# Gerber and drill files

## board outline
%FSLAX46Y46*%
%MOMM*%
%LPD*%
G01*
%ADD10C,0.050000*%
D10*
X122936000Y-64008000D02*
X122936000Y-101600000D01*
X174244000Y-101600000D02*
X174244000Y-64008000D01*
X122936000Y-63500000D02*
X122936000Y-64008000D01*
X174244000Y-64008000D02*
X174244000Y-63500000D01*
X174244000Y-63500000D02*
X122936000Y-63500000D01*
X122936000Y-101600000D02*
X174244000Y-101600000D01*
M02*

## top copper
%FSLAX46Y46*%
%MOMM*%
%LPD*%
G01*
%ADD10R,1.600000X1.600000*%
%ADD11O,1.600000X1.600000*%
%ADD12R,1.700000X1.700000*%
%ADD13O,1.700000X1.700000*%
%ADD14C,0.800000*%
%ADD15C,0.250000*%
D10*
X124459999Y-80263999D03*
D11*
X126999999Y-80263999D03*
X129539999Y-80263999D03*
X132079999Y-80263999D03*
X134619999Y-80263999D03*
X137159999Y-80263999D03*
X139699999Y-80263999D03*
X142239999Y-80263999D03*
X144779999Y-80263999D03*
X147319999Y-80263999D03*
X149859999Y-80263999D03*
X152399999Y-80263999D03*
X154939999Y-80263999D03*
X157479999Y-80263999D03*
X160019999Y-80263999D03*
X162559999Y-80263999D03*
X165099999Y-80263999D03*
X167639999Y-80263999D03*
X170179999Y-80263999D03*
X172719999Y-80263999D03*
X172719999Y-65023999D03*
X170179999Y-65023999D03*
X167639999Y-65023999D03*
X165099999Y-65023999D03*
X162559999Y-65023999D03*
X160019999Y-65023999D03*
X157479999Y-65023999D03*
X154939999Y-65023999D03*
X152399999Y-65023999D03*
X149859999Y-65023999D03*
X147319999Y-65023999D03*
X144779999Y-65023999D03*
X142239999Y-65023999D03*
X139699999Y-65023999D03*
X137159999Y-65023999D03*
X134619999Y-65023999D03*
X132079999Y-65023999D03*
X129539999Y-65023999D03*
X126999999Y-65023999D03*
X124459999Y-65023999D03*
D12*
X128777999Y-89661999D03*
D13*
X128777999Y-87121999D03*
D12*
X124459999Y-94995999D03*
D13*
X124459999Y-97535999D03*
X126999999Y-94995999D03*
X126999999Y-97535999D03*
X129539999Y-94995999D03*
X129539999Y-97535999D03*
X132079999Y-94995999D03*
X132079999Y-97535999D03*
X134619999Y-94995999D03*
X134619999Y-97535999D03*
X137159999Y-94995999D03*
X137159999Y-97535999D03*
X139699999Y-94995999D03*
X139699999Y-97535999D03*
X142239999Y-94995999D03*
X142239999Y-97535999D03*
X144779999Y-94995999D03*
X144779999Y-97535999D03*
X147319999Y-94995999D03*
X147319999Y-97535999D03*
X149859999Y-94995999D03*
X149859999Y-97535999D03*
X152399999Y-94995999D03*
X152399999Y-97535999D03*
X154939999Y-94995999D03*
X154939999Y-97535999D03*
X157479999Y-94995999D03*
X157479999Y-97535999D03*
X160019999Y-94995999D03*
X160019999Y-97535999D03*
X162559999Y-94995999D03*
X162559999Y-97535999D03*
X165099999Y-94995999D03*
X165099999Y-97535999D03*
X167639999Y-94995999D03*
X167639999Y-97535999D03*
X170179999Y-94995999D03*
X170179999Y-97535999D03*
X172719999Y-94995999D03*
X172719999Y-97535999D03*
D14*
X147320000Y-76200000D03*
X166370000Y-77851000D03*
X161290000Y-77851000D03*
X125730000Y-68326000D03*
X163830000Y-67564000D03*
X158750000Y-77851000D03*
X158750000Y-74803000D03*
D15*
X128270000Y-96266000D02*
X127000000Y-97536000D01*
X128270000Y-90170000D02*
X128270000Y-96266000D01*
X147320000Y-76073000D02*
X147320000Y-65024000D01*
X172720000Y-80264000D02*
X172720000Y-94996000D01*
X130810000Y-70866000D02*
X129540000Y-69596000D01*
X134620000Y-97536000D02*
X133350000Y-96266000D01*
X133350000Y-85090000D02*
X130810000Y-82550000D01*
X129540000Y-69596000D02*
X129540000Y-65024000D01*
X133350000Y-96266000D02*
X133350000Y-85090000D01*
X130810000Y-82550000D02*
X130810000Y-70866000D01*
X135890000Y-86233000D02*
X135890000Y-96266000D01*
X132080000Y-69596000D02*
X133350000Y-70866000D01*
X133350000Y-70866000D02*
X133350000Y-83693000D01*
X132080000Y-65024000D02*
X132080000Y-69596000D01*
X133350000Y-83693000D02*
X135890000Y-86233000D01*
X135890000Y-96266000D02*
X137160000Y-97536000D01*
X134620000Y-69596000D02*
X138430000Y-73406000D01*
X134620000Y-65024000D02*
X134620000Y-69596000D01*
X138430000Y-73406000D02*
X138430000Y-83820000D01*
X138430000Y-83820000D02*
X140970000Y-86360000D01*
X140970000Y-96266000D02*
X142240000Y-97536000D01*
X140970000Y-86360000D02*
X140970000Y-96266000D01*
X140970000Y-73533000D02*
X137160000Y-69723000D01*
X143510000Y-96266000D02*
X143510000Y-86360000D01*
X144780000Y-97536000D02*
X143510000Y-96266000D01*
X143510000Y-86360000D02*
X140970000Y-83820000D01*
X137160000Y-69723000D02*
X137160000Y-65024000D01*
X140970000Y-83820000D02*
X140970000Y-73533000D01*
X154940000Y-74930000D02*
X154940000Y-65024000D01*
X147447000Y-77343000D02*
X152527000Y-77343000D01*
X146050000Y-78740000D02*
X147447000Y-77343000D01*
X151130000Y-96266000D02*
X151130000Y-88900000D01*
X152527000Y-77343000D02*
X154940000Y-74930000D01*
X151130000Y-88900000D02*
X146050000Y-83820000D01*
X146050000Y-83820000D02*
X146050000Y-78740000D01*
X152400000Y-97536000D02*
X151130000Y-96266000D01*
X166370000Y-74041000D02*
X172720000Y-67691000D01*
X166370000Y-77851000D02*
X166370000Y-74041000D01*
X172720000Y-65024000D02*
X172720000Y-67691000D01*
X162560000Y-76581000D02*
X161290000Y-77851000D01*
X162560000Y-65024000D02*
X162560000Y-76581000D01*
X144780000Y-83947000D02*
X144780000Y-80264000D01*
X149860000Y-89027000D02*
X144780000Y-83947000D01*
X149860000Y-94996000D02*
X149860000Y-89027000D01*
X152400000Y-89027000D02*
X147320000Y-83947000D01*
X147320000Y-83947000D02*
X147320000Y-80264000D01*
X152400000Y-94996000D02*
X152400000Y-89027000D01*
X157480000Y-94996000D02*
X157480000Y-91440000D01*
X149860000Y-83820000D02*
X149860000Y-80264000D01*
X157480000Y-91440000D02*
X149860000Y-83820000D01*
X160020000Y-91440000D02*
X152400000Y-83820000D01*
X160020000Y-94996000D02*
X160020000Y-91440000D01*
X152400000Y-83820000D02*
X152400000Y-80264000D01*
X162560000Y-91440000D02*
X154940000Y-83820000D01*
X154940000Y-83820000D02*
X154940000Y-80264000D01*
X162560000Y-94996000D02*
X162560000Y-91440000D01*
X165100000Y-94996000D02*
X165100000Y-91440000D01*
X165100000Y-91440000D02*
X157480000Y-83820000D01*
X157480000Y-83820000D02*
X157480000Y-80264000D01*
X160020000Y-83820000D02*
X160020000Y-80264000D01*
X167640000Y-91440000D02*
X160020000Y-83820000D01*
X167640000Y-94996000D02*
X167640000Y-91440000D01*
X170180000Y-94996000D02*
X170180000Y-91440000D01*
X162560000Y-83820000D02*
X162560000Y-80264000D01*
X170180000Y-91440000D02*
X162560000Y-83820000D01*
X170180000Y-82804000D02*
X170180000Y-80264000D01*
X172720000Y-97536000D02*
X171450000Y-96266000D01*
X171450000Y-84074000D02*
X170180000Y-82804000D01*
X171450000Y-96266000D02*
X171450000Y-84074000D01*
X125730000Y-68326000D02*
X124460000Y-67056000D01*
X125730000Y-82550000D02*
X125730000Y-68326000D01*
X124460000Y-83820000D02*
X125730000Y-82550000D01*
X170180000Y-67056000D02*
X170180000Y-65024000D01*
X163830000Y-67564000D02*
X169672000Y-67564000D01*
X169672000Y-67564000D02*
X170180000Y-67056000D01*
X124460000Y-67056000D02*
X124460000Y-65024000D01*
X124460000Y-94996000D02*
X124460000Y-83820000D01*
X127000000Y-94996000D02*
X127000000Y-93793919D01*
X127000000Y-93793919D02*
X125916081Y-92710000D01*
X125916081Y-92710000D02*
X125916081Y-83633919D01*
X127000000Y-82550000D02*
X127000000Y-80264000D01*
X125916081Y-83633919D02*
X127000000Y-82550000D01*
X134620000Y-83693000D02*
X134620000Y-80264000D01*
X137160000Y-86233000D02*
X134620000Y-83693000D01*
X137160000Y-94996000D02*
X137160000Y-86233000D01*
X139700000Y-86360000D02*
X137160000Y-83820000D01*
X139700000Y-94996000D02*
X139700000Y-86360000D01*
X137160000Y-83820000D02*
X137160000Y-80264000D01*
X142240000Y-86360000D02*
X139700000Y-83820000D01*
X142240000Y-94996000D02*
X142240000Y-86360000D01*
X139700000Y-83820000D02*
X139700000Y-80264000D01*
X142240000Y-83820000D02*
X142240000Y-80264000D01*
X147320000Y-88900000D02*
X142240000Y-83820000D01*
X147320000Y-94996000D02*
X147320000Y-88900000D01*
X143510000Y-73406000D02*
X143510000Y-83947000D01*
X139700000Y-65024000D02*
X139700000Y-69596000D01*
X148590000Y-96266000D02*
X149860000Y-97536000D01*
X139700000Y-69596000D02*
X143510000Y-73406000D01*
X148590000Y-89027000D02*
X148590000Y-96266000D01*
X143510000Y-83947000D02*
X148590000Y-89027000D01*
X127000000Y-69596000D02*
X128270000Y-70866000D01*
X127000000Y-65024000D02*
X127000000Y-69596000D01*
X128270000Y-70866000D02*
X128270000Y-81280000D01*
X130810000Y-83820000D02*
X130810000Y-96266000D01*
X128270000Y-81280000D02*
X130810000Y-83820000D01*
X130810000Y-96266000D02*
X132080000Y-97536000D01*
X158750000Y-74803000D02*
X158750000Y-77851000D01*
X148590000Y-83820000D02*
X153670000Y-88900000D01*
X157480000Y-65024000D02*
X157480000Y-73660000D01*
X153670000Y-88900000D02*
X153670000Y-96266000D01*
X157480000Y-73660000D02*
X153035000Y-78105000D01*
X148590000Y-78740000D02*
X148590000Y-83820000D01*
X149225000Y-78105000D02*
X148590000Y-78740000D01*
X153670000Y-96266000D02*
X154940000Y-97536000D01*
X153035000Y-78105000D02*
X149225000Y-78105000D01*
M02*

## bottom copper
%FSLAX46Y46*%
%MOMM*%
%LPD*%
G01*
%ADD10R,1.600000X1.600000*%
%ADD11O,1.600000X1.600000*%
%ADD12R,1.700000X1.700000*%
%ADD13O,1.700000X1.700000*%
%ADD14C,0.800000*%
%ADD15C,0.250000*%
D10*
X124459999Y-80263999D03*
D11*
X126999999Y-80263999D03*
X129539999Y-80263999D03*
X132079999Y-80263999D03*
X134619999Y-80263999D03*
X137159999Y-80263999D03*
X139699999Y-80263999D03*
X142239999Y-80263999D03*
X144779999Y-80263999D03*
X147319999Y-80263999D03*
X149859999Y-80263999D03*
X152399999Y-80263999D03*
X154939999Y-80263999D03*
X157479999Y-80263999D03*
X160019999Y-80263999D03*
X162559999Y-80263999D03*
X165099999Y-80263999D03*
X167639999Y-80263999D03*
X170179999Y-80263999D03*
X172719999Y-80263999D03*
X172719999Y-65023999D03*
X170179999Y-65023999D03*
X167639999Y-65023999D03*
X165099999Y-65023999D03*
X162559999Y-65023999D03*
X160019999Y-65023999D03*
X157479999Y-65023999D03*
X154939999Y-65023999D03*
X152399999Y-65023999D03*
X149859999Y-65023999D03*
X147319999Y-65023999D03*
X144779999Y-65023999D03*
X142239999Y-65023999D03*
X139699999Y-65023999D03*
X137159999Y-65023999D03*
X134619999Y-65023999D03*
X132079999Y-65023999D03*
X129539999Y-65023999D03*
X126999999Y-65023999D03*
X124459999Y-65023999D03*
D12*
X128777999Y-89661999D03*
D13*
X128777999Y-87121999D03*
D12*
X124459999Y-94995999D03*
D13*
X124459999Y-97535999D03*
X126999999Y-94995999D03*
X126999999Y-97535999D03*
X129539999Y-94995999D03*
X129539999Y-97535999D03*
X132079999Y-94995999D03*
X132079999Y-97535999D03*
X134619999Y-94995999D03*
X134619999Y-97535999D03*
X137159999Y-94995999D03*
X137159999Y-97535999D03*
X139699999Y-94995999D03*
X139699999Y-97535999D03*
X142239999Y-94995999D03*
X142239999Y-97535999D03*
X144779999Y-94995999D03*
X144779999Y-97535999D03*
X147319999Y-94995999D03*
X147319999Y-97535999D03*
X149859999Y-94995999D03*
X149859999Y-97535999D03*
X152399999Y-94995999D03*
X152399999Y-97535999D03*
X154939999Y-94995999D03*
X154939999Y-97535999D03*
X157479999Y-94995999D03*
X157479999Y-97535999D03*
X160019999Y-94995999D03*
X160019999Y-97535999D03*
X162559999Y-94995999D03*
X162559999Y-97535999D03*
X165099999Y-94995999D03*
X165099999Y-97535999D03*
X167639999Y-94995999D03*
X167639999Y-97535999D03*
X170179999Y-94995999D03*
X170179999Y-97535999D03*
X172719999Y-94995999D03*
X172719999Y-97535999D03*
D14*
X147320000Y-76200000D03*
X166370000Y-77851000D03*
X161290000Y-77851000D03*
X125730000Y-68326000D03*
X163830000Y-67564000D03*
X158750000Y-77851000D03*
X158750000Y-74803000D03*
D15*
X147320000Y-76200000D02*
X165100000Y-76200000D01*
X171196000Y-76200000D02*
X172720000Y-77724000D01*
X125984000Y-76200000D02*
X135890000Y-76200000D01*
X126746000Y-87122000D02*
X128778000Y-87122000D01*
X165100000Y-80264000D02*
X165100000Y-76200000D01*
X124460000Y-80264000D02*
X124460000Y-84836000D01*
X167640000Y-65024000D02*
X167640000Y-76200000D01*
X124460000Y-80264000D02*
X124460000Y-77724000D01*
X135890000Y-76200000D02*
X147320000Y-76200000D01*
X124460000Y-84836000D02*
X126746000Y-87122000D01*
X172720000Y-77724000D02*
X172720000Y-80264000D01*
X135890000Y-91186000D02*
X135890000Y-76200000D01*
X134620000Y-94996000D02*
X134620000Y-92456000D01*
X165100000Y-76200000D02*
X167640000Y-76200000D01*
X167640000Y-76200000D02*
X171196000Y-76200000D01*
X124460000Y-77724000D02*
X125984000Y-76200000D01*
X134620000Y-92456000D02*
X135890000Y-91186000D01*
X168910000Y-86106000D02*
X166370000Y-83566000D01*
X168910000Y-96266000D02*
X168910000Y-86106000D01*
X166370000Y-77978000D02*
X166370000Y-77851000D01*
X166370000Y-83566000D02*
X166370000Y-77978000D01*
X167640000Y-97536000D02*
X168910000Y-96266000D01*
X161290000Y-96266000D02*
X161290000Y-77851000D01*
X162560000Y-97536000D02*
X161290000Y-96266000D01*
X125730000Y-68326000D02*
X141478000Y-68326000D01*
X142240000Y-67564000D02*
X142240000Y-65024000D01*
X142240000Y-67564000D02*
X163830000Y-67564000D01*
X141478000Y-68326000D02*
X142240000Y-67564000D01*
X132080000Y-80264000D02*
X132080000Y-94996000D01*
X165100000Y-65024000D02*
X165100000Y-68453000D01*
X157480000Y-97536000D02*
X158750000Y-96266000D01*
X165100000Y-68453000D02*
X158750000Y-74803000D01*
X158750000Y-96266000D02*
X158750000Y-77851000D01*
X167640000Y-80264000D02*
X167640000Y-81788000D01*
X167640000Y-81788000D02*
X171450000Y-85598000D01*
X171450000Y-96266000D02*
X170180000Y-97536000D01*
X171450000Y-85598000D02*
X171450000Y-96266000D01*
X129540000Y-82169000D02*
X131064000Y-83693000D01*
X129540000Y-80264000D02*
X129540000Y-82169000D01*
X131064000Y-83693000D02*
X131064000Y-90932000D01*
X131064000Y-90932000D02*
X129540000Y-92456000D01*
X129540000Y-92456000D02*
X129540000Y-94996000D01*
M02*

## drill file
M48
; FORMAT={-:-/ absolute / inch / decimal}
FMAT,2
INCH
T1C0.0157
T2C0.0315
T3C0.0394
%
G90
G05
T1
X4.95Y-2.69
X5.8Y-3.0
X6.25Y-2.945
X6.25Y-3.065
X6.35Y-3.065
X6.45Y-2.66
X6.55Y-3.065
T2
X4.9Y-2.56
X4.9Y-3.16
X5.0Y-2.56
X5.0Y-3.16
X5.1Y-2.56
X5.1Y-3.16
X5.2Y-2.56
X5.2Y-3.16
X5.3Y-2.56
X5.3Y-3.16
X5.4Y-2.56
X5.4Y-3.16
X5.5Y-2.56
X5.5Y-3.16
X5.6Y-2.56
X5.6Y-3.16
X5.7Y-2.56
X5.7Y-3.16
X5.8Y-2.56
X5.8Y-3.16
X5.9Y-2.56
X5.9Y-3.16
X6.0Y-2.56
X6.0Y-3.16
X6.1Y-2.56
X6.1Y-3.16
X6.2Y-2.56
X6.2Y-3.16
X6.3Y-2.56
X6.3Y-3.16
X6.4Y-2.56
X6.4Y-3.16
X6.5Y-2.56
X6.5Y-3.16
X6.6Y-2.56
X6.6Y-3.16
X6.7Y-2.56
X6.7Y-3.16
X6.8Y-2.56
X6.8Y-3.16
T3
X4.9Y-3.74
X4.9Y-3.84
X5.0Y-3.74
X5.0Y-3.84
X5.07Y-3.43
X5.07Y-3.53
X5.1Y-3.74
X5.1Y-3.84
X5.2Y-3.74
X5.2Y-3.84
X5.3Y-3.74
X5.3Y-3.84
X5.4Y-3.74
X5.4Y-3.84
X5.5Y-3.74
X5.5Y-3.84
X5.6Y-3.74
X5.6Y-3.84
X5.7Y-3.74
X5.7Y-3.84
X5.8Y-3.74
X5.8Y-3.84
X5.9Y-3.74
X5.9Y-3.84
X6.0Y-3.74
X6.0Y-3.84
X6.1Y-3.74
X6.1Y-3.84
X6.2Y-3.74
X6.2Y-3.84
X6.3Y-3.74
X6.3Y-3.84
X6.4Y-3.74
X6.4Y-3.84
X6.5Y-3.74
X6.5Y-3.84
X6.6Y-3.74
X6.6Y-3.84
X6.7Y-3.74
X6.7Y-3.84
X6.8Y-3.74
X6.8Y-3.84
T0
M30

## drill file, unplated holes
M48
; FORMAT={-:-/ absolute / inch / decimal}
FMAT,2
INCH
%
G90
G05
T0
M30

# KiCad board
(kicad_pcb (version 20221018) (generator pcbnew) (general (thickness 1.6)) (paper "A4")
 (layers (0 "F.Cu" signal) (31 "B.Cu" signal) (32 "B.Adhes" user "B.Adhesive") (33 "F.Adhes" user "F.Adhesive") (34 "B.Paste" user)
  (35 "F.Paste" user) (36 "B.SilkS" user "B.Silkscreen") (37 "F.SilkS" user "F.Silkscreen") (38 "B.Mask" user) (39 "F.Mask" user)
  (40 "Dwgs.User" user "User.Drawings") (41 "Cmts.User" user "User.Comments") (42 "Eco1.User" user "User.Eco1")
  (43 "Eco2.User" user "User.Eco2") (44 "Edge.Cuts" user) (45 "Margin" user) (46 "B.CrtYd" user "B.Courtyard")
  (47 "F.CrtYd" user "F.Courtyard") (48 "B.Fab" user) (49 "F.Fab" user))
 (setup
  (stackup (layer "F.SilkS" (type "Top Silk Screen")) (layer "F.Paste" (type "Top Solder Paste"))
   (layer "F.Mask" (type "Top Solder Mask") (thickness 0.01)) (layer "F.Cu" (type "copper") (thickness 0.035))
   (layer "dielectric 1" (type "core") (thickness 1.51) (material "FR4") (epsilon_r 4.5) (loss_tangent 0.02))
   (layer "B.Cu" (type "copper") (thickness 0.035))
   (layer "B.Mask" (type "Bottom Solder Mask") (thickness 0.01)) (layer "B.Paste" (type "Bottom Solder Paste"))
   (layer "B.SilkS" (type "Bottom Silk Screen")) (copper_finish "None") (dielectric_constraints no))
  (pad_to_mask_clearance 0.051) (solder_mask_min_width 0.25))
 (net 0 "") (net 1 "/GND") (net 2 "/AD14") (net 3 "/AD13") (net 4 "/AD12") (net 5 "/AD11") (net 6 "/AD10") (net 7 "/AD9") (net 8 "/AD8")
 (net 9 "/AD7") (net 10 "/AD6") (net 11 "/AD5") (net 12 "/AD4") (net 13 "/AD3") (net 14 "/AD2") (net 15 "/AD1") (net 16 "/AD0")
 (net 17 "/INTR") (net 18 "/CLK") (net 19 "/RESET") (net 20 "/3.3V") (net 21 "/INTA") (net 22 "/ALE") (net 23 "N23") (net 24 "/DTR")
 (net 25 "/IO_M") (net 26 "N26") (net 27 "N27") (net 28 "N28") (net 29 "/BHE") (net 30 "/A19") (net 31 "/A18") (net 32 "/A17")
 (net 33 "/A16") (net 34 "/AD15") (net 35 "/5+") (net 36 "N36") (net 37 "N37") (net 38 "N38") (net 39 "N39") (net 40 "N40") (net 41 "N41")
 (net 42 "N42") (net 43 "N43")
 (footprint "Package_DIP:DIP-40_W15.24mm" (layer "F.Cu") (at 124.46 80.264 90)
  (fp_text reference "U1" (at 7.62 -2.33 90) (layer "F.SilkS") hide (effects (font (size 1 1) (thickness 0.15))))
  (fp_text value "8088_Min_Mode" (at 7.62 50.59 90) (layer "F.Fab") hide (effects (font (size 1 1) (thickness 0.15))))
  (pad "1" thru_hole rect (at 0 0 90) (size 1.6 1.6) (drill 0.8) (layers "*.Cu" "*.Mask") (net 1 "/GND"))
  (pad "2" thru_hole oval (at 0 2.54 90) (size 1.6 1.6) (drill 0.8) (layers "*.Cu" "*.Mask") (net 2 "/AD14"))
  (pad "3" thru_hole oval (at 0 5.08 90) (size 1.6 1.6) (drill 0.8) (layers "*.Cu" "*.Mask") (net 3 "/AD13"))
  (pad "4" thru_hole oval (at 0 7.62 90) (size 1.6 1.6) (drill 0.8) (layers "*.Cu" "*.Mask") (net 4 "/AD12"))
  (pad "5" thru_hole oval (at 0 10.16 90) (size 1.6 1.6) (drill 0.8) (layers "*.Cu" "*.Mask") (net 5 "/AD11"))
  (pad "6" thru_hole oval (at 0 12.7 90) (size 1.6 1.6) (drill 0.8) (layers "*.Cu" "*.Mask") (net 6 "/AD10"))
  (pad "7" thru_hole oval (at 0 15.24 90) (size 1.6 1.6) (drill 0.8) (layers "*.Cu" "*.Mask") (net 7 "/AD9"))
  (pad "8" thru_hole oval (at 0 17.78 90) (size 1.6 1.6) (drill 0.8) (layers "*.Cu" "*.Mask") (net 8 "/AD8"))
  (pad "9" thru_hole oval (at 0 20.32 90) (size 1.6 1.6) (drill 0.8) (layers "*.Cu" "*.Mask") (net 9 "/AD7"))
  (pad "10" thru_hole oval (at 0 22.86 90) (size 1.6 1.6) (drill 0.8) (layers "*.Cu" "*.Mask") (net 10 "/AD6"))
  (pad "11" thru_hole oval (at 0 25.4 90) (size 1.6 1.6) (drill 0.8) (layers "*.Cu" "*.Mask") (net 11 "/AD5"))
  (pad "12" thru_hole oval (at 0 27.94 90) (size 1.6 1.6) (drill 0.8) (layers "*.Cu" "*.Mask") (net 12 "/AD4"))
  (pad "13" thru_hole oval (at 0 30.48 90) (size 1.6 1.6) (drill 0.8) (layers "*.Cu" "*.Mask") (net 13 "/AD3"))
  (pad "14" thru_hole oval (at 0 33.02 90) (size 1.6 1.6) (drill 0.8) (layers "*.Cu" "*.Mask") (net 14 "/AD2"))
  (pad "15" thru_hole oval (at 0 35.56 90) (size 1.6 1.6) (drill 0.8) (layers "*.Cu" "*.Mask") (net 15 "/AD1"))
  (pad "16" thru_hole oval (at 0 38.1 90) (size 1.6 1.6) (drill 0.8) (layers "*.Cu" "*.Mask") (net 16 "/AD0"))
  (pad "17" thru_hole oval (at 0 40.64 90) (size 1.6 1.6) (drill 0.8) (layers "*.Cu" "*.Mask") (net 1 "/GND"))
  (pad "18" thru_hole oval (at 0 43.18 90) (size 1.6 1.6) (drill 0.8) (layers "*.Cu" "*.Mask") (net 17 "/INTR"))
  (pad "19" thru_hole oval (at 0 45.72 90) (size 1.6 1.6) (drill 0.8) (layers "*.Cu" "*.Mask") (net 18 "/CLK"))
  (pad "20" thru_hole oval (at 0 48.26 90) (size 1.6 1.6) (drill 0.8) (layers "*.Cu" "*.Mask") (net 1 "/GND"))
  (pad "21" thru_hole oval (at 15.24 48.26 90) (size 1.6 1.6) (drill 0.8) (layers "*.Cu" "*.Mask") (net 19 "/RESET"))
  (pad "22" thru_hole oval (at 15.24 45.72 90) (size 1.6 1.6) (drill 0.8) (layers "*.Cu" "*.Mask") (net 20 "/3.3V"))
  (pad "23" thru_hole oval (at 15.24 43.18 90) (size 1.6 1.6) (drill 0.8) (layers "*.Cu" "*.Mask") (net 1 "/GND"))
  (pad "24" thru_hole oval (at 15.24 40.64 90) (size 1.6 1.6) (drill 0.8) (layers "*.Cu" "*.Mask") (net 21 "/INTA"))
  (pad "25" thru_hole oval (at 15.24 38.1 90) (size 1.6 1.6) (drill 0.8) (layers "*.Cu" "*.Mask") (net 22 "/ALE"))
  (pad "26" thru_hole oval (at 15.24 35.56 90) (size 1.6 1.6) (drill 0.8) (layers "*.Cu" "*.Mask") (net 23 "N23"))
  (pad "27" thru_hole oval (at 15.24 33.02 90) (size 1.6 1.6) (drill 0.8) (layers "*.Cu" "*.Mask") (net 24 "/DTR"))
  (pad "28" thru_hole oval (at 15.24 30.48 90) (size 1.6 1.6) (drill 0.8) (layers "*.Cu" "*.Mask") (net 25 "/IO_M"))
  (pad "29" thru_hole oval (at 15.24 27.94 90) (size 1.6 1.6) (drill 0.8) (layers "*.Cu" "*.Mask") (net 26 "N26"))
  (pad "30" thru_hole oval (at 15.24 25.4 90) (size 1.6 1.6) (drill 0.8) (layers "*.Cu" "*.Mask") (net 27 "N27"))
  (pad "31" thru_hole oval (at 15.24 22.86 90) (size 1.6 1.6) (drill 0.8) (layers "*.Cu" "*.Mask") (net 1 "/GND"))
  (pad "32" thru_hole oval (at 15.24 20.32 90) (size 1.6 1.6) (drill 0.8) (layers "*.Cu" "*.Mask") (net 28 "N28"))
  (pad "33" thru_hole oval (at 15.24 17.78 90) (size 1.6 1.6) (drill 0.8) (layers "*.Cu" "*.Mask") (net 20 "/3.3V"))
  (pad "34" thru_hole oval (at 15.24 15.24 90) (size 1.6 1.6) (drill 0.8) (layers "*.Cu" "*.Mask") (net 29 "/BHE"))
  (pad "35" thru_hole oval (at 15.24 12.7 90) (size 1.6 1.6) (drill 0.8) (layers "*.Cu" "*.Mask") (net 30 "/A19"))
  (pad "36" thru_hole oval (at 15.24 10.16 90) (size 1.6 1.6) (drill 0.8) (layers "*.Cu" "*.Mask") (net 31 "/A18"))
  (pad "37" thru_hole oval (at 15.24 7.62 90) (size 1.6 1.6) (drill 0.8) (layers "*.Cu" "*.Mask") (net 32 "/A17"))
  (pad "38" thru_hole oval (at 15.24 5.08 90) (size 1.6 1.6) (drill 0.8) (layers "*.Cu" "*.Mask") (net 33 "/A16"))
  (pad "39" thru_hole oval (at 15.24 2.54 90) (size 1.6 1.6) (drill 0.8) (layers "*.Cu" "*.Mask") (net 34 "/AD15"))
  (pad "40" thru_hole oval (at 15.24 0 90) (size 1.6 1.6) (drill 0.8) (layers "*.Cu" "*.Mask") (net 20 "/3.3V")))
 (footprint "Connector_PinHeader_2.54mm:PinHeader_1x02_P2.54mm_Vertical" (layer "F.Cu") (at 128.778 89.662 180)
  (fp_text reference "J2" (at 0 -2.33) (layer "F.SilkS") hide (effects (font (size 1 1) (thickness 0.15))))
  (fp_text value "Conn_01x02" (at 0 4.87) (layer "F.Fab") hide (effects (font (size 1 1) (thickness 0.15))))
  (pad "1" thru_hole rect (at 0 0 180) (size 1.7 1.7) (drill 1) (layers "*.Cu" "*.Mask") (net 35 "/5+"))
  (pad "2" thru_hole oval (at 0 2.54 180) (size 1.7 1.7) (drill 1) (layers "*.Cu" "*.Mask") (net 1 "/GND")))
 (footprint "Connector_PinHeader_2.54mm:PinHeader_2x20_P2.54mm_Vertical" (layer "B.Cu") (at 124.46 94.996 -90)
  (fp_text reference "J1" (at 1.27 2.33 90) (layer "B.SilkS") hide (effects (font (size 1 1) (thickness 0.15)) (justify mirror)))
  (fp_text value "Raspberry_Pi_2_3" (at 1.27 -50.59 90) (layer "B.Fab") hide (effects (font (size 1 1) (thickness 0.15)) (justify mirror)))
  (pad "1" thru_hole rect (at 0 0 270) (size 1.7 1.7) (drill 1) (layers "*.Cu" "*.Mask") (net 20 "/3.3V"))
  (pad "2" thru_hole oval (at 2.54 0 270) (size 1.7 1.7) (drill 1) (layers "*.Cu" "*.Mask") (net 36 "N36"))
  (pad "3" thru_hole oval (at 0 -2.54 270) (size 1.7 1.7) (drill 1) (layers "*.Cu" "*.Mask") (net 2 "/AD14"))
  (pad "4" thru_hole oval (at 2.54 -2.54 270) (size 1.7 1.7) (drill 1) (layers "*.Cu" "*.Mask") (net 35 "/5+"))
  (pad "5" thru_hole oval (at 0 -5.08 270) (size 1.7 1.7) (drill 1) (layers "*.Cu" "*.Mask") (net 3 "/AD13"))
  (pad "6" thru_hole oval (at 2.54 -5.08 270) (size 1.7 1.7) (drill 1) (layers "*.Cu" "*.Mask") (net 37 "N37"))
  (pad "7" thru_hole oval (at 0 -7.62 270) (size 1.7 1.7) (drill 1) (layers "*.Cu" "*.Mask") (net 4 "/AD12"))
  (pad "8" thru_hole oval (at 2.54 -7.62 270) (size 1.7 1.7) (drill 1) (layers "*.Cu" "*.Mask") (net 34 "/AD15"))
  (pad "9" thru_hole oval (at 0 -10.16 270) (size 1.7 1.7) (drill 1) (layers "*.Cu" "*.Mask") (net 1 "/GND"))
  (pad "10" thru_hole oval (at 2.54 -10.16 270) (size 1.7 1.7) (drill 1) (layers "*.Cu" "*.Mask") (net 33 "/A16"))
  (pad "11" thru_hole oval (at 0 -12.7 270) (size 1.7 1.7) (drill 1) (layers "*.Cu" "*.Mask") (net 5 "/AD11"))
  (pad "12" thru_hole oval (at 2.54 -12.7 270) (size 1.7 1.7) (drill 1) (layers "*.Cu" "*.Mask") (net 32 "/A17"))
  (pad "13" thru_hole oval (at 0 -15.24 270) (size 1.7 1.7) (drill 1) (layers "*.Cu" "*.Mask") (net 6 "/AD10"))
  (pad "14" thru_hole oval (at 2.54 -15.24 270) (size 1.7 1.7) (drill 1) (layers "*.Cu" "*.Mask") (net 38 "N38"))
  (pad "15" thru_hole oval (at 0 -17.78 270) (size 1.7 1.7) (drill 1) (layers "*.Cu" "*.Mask") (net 7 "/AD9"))
  (pad "16" thru_hole oval (at 2.54 -17.78 270) (size 1.7 1.7) (drill 1) (layers "*.Cu" "*.Mask") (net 31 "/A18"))
  (pad "17" thru_hole oval (at 0 -20.32 270) (size 1.7 1.7) (drill 1) (layers "*.Cu" "*.Mask") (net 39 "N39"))
  (pad "18" thru_hole oval (at 2.54 -20.32 270) (size 1.7 1.7) (drill 1) (layers "*.Cu" "*.Mask") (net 30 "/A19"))
  (pad "19" thru_hole oval (at 0 -22.86 270) (size 1.7 1.7) (drill 1) (layers "*.Cu" "*.Mask") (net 8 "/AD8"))
  (pad "20" thru_hole oval (at 2.54 -22.86 270) (size 1.7 1.7) (drill 1) (layers "*.Cu" "*.Mask") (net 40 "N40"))
  (pad "21" thru_hole oval (at 0 -25.4 270) (size 1.7 1.7) (drill 1) (layers "*.Cu" "*.Mask") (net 9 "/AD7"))
  (pad "22" thru_hole oval (at 2.54 -25.4 270) (size 1.7 1.7) (drill 1) (layers "*.Cu" "*.Mask") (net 29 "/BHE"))
  (pad "23" thru_hole oval (at 0 -27.94 270) (size 1.7 1.7) (drill 1) (layers "*.Cu" "*.Mask") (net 10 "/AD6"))
  (pad "24" thru_hole oval (at 2.54 -27.94 270) (size 1.7 1.7) (drill 1) (layers "*.Cu" "*.Mask") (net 25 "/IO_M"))
  (pad "25" thru_hole oval (at 0 -30.48 270) (size 1.7 1.7) (drill 1) (layers "*.Cu" "*.Mask") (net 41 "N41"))
  (pad "26" thru_hole oval (at 2.54 -30.48 270) (size 1.7 1.7) (drill 1) (layers "*.Cu" "*.Mask") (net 24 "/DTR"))
  (pad "27" thru_hole oval (at 0 -33.02 270) (size 1.7 1.7) (drill 1) (layers "*.Cu" "*.Mask") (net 11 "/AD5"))
  (pad "28" thru_hole oval (at 2.54 -33.02 270) (size 1.7 1.7) (drill 1) (layers "*.Cu" "*.Mask") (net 21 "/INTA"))
  (pad "29" thru_hole oval (at 0 -35.56 270) (size 1.7 1.7) (drill 1) (layers "*.Cu" "*.Mask") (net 12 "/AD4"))
  (pad "30" thru_hole oval (at 2.54 -35.56 270) (size 1.7 1.7) (drill 1) (layers "*.Cu" "*.Mask") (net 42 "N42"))
  (pad "31" thru_hole oval (at 0 -38.1 270) (size 1.7 1.7) (drill 1) (layers "*.Cu" "*.Mask") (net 13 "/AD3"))
  (pad "32" thru_hole oval (at 2.54 -38.1 270) (size 1.7 1.7) (drill 1) (layers "*.Cu" "*.Mask") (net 22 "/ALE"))
  (pad "33" thru_hole oval (at 0 -40.64 270) (size 1.7 1.7) (drill 1) (layers "*.Cu" "*.Mask") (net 14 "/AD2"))
  (pad "34" thru_hole oval (at 2.54 -40.64 270) (size 1.7 1.7) (drill 1) (layers "*.Cu" "*.Mask") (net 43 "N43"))
  (pad "35" thru_hole oval (at 0 -43.18 270) (size 1.7 1.7) (drill 1) (layers "*.Cu" "*.Mask") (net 15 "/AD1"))
  (pad "36" thru_hole oval (at 2.54 -43.18 270) (size 1.7 1.7) (drill 1) (layers "*.Cu" "*.Mask") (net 19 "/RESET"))
  (pad "37" thru_hole oval (at 0 -45.72 270) (size 1.7 1.7) (drill 1) (layers "*.Cu" "*.Mask") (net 16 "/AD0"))
  (pad "38" thru_hole oval (at 2.54 -45.72 270) (size 1.7 1.7) (drill 1) (layers "*.Cu" "*.Mask") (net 17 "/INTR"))
  (pad "39" thru_hole oval (at 0 -48.26 270) (size 1.7 1.7) (drill 1) (layers "*.Cu" "*.Mask") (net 1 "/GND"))
  (pad "40" thru_hole oval (at 2.54 -48.26 270) (size 1.7 1.7) (drill 1) (layers "*.Cu" "*.Mask") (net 18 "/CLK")))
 (gr_line (start 122.936 64.008) (end 122.936 101.6) (stroke (width 0.05) (type solid)) (layer "Edge.Cuts"))
 (gr_line (start 174.244 101.6) (end 174.244 64.008) (stroke (width 0.05) (type solid)) (layer "Edge.Cuts"))
 (gr_line (start 122.936 63.5) (end 122.936 64.008) (stroke (width 0.05) (type solid)) (layer "Edge.Cuts"))
 (gr_line (start 174.244 64.008) (end 174.244 63.5) (stroke (width 0.05) (type solid)) (layer "Edge.Cuts"))
 (gr_line (start 174.244 63.5) (end 122.936 63.5) (stroke (width 0.05) (type solid)) (layer "Edge.Cuts"))
 (gr_line (start 122.936 101.6) (end 174.244 101.6) (stroke (width 0.05) (type solid)) (layer "Edge.Cuts"))
 (segment (start 128.27 96.266) (end 127 97.536) (width 0.25) (layer "F.Cu") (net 35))
 (segment (start 128.27 90.17) (end 128.27 96.266) (width 0.25) (layer "F.Cu") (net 35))
 (segment (start 147.32 76.073) (end 147.32 65.024) (width 0.25) (layer "F.Cu") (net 1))
 (segment (start 172.72 80.264) (end 172.72 94.996) (width 0.25) (layer "F.Cu") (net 1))
 (via (at 147.32 76.2) (size 0.8) (drill 0.4) (layers "F.Cu" "B.Cu") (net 1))
 (segment (start 147.32 76.2) (end 165.1 76.2) (width 0.25) (layer "B.Cu") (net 1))
 (segment (start 171.196 76.2) (end 172.72 77.724) (width 0.25) (layer "B.Cu") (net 1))
 (segment (start 125.984 76.2) (end 135.89 76.2) (width 0.25) (layer "B.Cu") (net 1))
 (segment (start 126.746 87.122) (end 128.778 87.122) (width 0.25) (layer "B.Cu") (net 1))
 (segment (start 165.1 80.264) (end 165.1 76.2) (width 0.25) (layer "B.Cu") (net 1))
 (segment (start 124.46 80.264) (end 124.46 84.836) (width 0.25) (layer "B.Cu") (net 1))
 (segment (start 167.64 65.024) (end 167.64 76.2) (width 0.25) (layer "B.Cu") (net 1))
 (segment (start 124.46 80.264) (end 124.46 77.724) (width 0.25) (layer "B.Cu") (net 1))
 (segment (start 135.89 76.2) (end 147.32 76.2) (width 0.25) (layer "B.Cu") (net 1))
 (segment (start 124.46 84.836) (end 126.746 87.122) (width 0.25) (layer "B.Cu") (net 1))
 (segment (start 172.72 77.724) (end 172.72 80.264) (width 0.25) (layer "B.Cu") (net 1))
 (segment (start 135.89 91.186) (end 135.89 76.2) (width 0.25) (layer "B.Cu") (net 1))
 (segment (start 134.62 94.996) (end 134.62 92.456) (width 0.25) (layer "B.Cu") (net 1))
 (segment (start 165.1 76.2) (end 167.64 76.2) (width 0.25) (layer "B.Cu") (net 1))
 (segment (start 167.64 76.2) (end 171.196 76.2) (width 0.25) (layer "B.Cu") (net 1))
 (segment (start 124.46 77.724) (end 125.984 76.2) (width 0.25) (layer "B.Cu") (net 1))
 (segment (start 134.62 92.456) (end 135.89 91.186) (width 0.25) (layer "B.Cu") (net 1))
 (segment (start 130.81 70.866) (end 129.54 69.596) (width 0.25) (layer "F.Cu") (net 33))
 (segment (start 134.62 97.536) (end 133.35 96.266) (width 0.25) (layer "F.Cu") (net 33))
 (segment (start 133.35 85.09) (end 130.81 82.55) (width 0.25) (layer "F.Cu") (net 33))
 (segment (start 129.54 69.596) (end 129.54 65.024) (width 0.25) (layer "F.Cu") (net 33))
 (segment (start 133.35 96.266) (end 133.35 85.09) (width 0.25) (layer "F.Cu") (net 33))
 (segment (start 130.81 82.55) (end 130.81 70.866) (width 0.25) (layer "F.Cu") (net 33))
 (segment (start 135.89 86.233) (end 135.89 96.266) (width 0.25) (layer "F.Cu") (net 32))
 (segment (start 132.08 69.596) (end 133.35 70.866) (width 0.25) (layer "F.Cu") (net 32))
 (segment (start 133.35 70.866) (end 133.35 83.693) (width 0.25) (layer "F.Cu") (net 32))
 (segment (start 132.08 65.024) (end 132.08 69.596) (width 0.25) (layer "F.Cu") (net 32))
 (segment (start 133.35 83.693) (end 135.89 86.233) (width 0.25) (layer "F.Cu") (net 32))
 (segment (start 135.89 96.266) (end 137.16 97.536) (width 0.25) (layer "F.Cu") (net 32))
 (segment (start 134.62 69.596) (end 138.43 73.406) (width 0.25) (layer "F.Cu") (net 31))
 (segment (start 134.62 65.024) (end 134.62 69.596) (width 0.25) (layer "F.Cu") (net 31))
 (segment (start 138.43 73.406) (end 138.43 83.82) (width 0.25) (layer "F.Cu") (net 31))
 (segment (start 138.43 83.82) (end 140.97 86.36) (width 0.25) (layer "F.Cu") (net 31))
 (segment (start 140.97 96.266) (end 142.24 97.536) (width 0.25) (layer "F.Cu") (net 31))
 (segment (start 140.97 86.36) (end 140.97 96.266) (width 0.25) (layer "F.Cu") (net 31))
 (segment (start 140.97 73.533) (end 137.16 69.723) (width 0.25) (layer "F.Cu") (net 30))
 (segment (start 143.51 96.266) (end 143.51 86.36) (width 0.25) (layer "F.Cu") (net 30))
 (segment (start 144.78 97.536) (end 143.51 96.266) (width 0.25) (layer "F.Cu") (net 30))
 (segment (start 143.51 86.36) (end 140.97 83.82) (width 0.25) (layer "F.Cu") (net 30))
 (segment (start 137.16 69.723) (end 137.16 65.024) (width 0.25) (layer "F.Cu") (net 30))
 (segment (start 140.97 83.82) (end 140.97 73.533) (width 0.25) (layer "F.Cu") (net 30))
 (segment (start 154.94 74.93) (end 154.94 65.024) (width 0.25) (layer "F.Cu") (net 25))
 (segment (start 147.447 77.343) (end 152.527 77.343) (width 0.25) (layer "F.Cu") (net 25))
 (segment (start 146.05 78.74) (end 147.447 77.343) (width 0.25) (layer "F.Cu") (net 25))
 (segment (start 151.13 96.266) (end 151.13 88.9) (width 0.25) (layer "F.Cu") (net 25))
 (segment (start 152.527 77.343) (end 154.94 74.93) (width 0.25) (layer "F.Cu") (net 25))
 (segment (start 151.13 88.9) (end 146.05 83.82) (width 0.25) (layer "F.Cu") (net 25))
 (segment (start 146.05 83.82) (end 146.05 78.74) (width 0.25) (layer "F.Cu") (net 25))
 (segment (start 152.4 97.536) (end 151.13 96.266) (width 0.25) (layer "F.Cu") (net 25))
 (segment (start 166.37 74.041) (end 172.72 67.691) (width 0.25) (layer "F.Cu") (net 19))
 (segment (start 166.37 77.851) (end 166.37 74.041) (width 0.25) (layer "F.Cu") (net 19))
 (segment (start 172.72 65.024) (end 172.72 67.691) (width 0.25) (layer "F.Cu") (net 19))
 (via (at 166.37 77.851) (size 0.8) (drill 0.4) (layers "F.Cu" "B.Cu") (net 19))
 (segment (start 168.91 86.106) (end 166.37 83.566) (width 0.25) (layer "B.Cu") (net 19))
 (segment (start 168.91 96.266) (end 168.91 86.106) (width 0.25) (layer "B.Cu") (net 19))
 (segment (start 166.37 77.978) (end 166.37 77.851) (width 0.25) (layer "B.Cu") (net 19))
 (segment (start 166.37 83.566) (end 166.37 77.978) (width 0.25) (layer "B.Cu") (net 19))
 (segment (start 167.64 97.536) (end 168.91 96.266) (width 0.25) (layer "B.Cu") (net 19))
 (segment (start 162.56 76.581) (end 161.29 77.851) (width 0.25) (layer "F.Cu") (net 22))
 (segment (start 162.56 65.024) (end 162.56 76.581) (width 0.25) (layer "F.Cu") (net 22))
 (via (at 161.29 77.851) (size 0.8) (drill 0.4) (layers "F.Cu" "B.Cu") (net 22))
 (segment (start 161.29 96.266) (end 161.29 77.851) (width 0.25) (layer "B.Cu") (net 22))
 (segment (start 162.56 97.536) (end 161.29 96.266) (width 0.25) (layer "B.Cu") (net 22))
 (segment (start 144.78 83.947) (end 144.78 80.264) (width 0.25) (layer "F.Cu") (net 9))
 (segment (start 149.86 89.027) (end 144.78 83.947) (width 0.25) (layer "F.Cu") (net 9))
 (segment (start 149.86 94.996) (end 149.86 89.027) (width 0.25) (layer "F.Cu") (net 9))
 (segment (start 152.4 89.027) (end 147.32 83.947) (width 0.25) (layer "F.Cu") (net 10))
 (segment (start 147.32 83.947) (end 147.32 80.264) (width 0.25) (layer "F.Cu") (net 10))
 (segment (start 152.4 94.996) (end 152.4 89.027) (width 0.25) (layer "F.Cu") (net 10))
 (segment (start 157.48 94.996) (end 157.48 91.44) (width 0.25) (layer "F.Cu") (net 11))
 (segment (start 149.86 83.82) (end 149.86 80.264) (width 0.25) (layer "F.Cu") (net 11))
 (segment (start 157.48 91.44) (end 149.86 83.82) (width 0.25) (layer "F.Cu") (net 11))
 (segment (start 160.02 91.44) (end 152.4 83.82) (width 0.25) (layer "F.Cu") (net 12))
 (segment (start 160.02 94.996) (end 160.02 91.44) (width 0.25) (layer "F.Cu") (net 12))
 (segment (start 152.4 83.82) (end 152.4 80.264) (width 0.25) (layer "F.Cu") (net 12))
 (segment (start 162.56 91.44) (end 154.94 83.82) (width 0.25) (layer "F.Cu") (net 13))
 (segment (start 154.94 83.82) (end 154.94 80.264) (width 0.25) (layer "F.Cu") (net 13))
 (segment (start 162.56 94.996) (end 162.56 91.44) (width 0.25) (layer "F.Cu") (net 13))
 (segment (start 165.1 94.996) (end 165.1 91.44) (width 0.25) (layer "F.Cu") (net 14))
 (segment (start 165.1 91.44) (end 157.48 83.82) (width 0.25) (layer "F.Cu") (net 14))
 (segment (start 157.48 83.82) (end 157.48 80.264) (width 0.25) (layer "F.Cu") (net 14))
 (segment (start 160.02 83.82) (end 160.02 80.264) (width 0.25) (layer "F.Cu") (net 15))
 (segment (start 167.64 91.44) (end 160.02 83.82) (width 0.25) (layer "F.Cu") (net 15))
 (segment (start 167.64 94.996) (end 167.64 91.44) (width 0.25) (layer "F.Cu") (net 15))
 (segment (start 170.18 94.996) (end 170.18 91.44) (width 0.25) (layer "F.Cu") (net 16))
 (segment (start 162.56 83.82) (end 162.56 80.264) (width 0.25) (layer "F.Cu") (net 16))
 (segment (start 170.18 91.44) (end 162.56 83.82) (width 0.25) (layer "F.Cu") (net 16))
 (segment (start 170.18 82.804) (end 170.18 80.264) (width 0.25) (layer "F.Cu") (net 18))
 (segment (start 172.72 97.536) (end 171.45 96.266) (width 0.25) (layer "F.Cu") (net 18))
 (segment (start 171.45 84.074) (end 170.18 82.804) (width 0.25) (layer "F.Cu") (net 18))
 (segment (start 171.45 96.266) (end 171.45 84.074) (width 0.25) (layer "F.Cu") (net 18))
 (segment (start 125.73 68.326) (end 124.46 67.056) (width 0.25) (layer "F.Cu") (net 20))
 (segment (start 125.73 82.55) (end 125.73 68.326) (width 0.25) (layer "F.Cu") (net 20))
 (segment (start 124.46 83.82) (end 125.73 82.55) (width 0.25) (layer "F.Cu") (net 20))
 (segment (start 170.18 67.056) (end 170.18 65.024) (width 0.25) (layer "F.Cu") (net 20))
 (segment (start 163.83 67.564) (end 169.672 67.564) (width 0.25) (layer "F.Cu") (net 20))
 (segment (start 169.672 67.564) (end 170.18 67.056) (width 0.25) (layer "F.Cu") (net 20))
 (segment (start 124.46 67.056) (end 124.46 65.024) (width 0.25) (layer "F.Cu") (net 20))
 (segment (start 124.46 94.996) (end 124.46 83.82) (width 0.25) (layer "F.Cu") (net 20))
 (via (at 125.73 68.326) (size 0.8) (drill 0.4) (layers "F.Cu" "B.Cu") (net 20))
 (via (at 163.83 67.564) (size 0.8) (drill 0.4) (layers "F.Cu" "B.Cu") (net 20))
 (segment (start 125.73 68.326) (end 141.478 68.326) (width 0.25) (layer "B.Cu") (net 20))
 (segment (start 142.24 67.564) (end 142.24 65.024) (width 0.25) (layer "B.Cu") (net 20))
 (segment (start 142.24 67.564) (end 163.83 67.564) (width 0.25) (layer "B.Cu") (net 20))
 (segment (start 141.478 68.326) (end 142.24 67.564) (width 0.25) (layer "B.Cu") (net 20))
 (segment (start 127 94.996) (end 127 93.793919) (width 0.25) (layer "F.Cu") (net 2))
 (segment (start 127 93.793919) (end 125.916081 92.71) (width 0.25) (layer "F.Cu") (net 2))
 (segment (start 125.916081 92.71) (end 125.916081 83.633919) (width 0.25) (layer "F.Cu") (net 2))
 (segment (start 127 82.55) (end 127 80.264) (width 0.25) (layer "F.Cu") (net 2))
 (segment (start 125.916081 83.633919) (end 127 82.55) (width 0.25) (layer "F.Cu") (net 2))
 (segment (start 132.08 80.264) (end 132.08 94.996) (width 0.25) (layer "B.Cu") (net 4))
 (segment (start 134.62 83.693) (end 134.62 80.264) (width 0.25) (layer "F.Cu") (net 5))
 (segment (start 137.16 86.233) (end 134.62 83.693) (width 0.25) (layer "F.Cu") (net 5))
 (segment (start 137.16 94.996) (end 137.16 86.233) (width 0.25) (layer "F.Cu") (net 5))
 (segment (start 139.7 86.36) (end 137.16 83.82) (width 0.25) (layer "F.Cu") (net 6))
 (segment (start 139.7 94.996) (end 139.7 86.36) (width 0.25) (layer "F.Cu") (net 6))
 (segment (start 137.16 83.82) (end 137.16 80.264) (width 0.25) (layer "F.Cu") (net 6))
 (segment (start 142.24 86.36) (end 139.7 83.82) (width 0.25) (layer "F.Cu") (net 7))
 (segment (start 142.24 94.996) (end 142.24 86.36) (width 0.25) (layer "F.Cu") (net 7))
 (segment (start 139.7 83.82) (end 139.7 80.264) (width 0.25) (layer "F.Cu") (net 7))
 (segment (start 142.24 83.82) (end 142.24 80.264) (width 0.25) (layer "F.Cu") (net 8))
 (segment (start 147.32 88.9) (end 142.24 83.82) (width 0.25) (layer "F.Cu") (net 8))
 (segment (start 147.32 94.996) (end 147.32 88.9) (width 0.25) (layer "F.Cu") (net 8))
 (segment (start 143.51 73.406) (end 143.51 83.947) (width 0.25) (layer "F.Cu") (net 29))
 (segment (start 139.7 65.024) (end 139.7 69.596) (width 0.25) (layer "F.Cu") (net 29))
 (segment (start 148.59 96.266) (end 149.86 97.536) (width 0.25) (layer "F.Cu") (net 29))
 (segment (start 139.7 69.596) (end 143.51 73.406) (width 0.25) (layer "F.Cu") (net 29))
 (segment (start 148.59 89.027) (end 148.59 96.266) (width 0.25) (layer "F.Cu") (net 29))
 (segment (start 143.51 83.947) (end 148.59 89.027) (width 0.25) (layer "F.Cu") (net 29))
 (segment (start 127 69.596) (end 128.27 70.866) (width 0.25) (layer "F.Cu") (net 34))
 (segment (start 127 65.024) (end 127 69.596) (width 0.25) (layer "F.Cu") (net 34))
 (segment (start 128.27 70.866) (end 128.27 81.28) (width 0.25) (layer "F.Cu") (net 34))
 (segment (start 130.81 83.82) (end 130.81 96.266) (width 0.25) (layer "F.Cu") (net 34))
 (segment (start 128.27 81.28) (end 130.81 83.82) (width 0.25) (layer "F.Cu") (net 34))
 (segment (start 130.81 96.266) (end 132.08 97.536) (width 0.25) (layer "F.Cu") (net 34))
 (segment (start 158.75 74.803) (end 158.75 77.851) (width 0.25) (layer "F.Cu") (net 21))
 (via (at 158.75 77.851) (size 0.8) (drill 0.4) (layers "F.Cu" "B.Cu") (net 21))
 (via (at 158.75 74.803) (size 0.8) (drill 0.4) (layers "F.Cu" "B.Cu") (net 21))
 (segment (start 165.1 65.024) (end 165.1 68.453) (width 0.25) (layer "B.Cu") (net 21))
 (segment (start 157.48 97.536) (end 158.75 96.266) (width 0.25) (layer "B.Cu") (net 21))
 (segment (start 165.1 68.453) (end 158.75 74.803) (width 0.25) (layer "B.Cu") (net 21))
 (segment (start 158.75 96.266) (end 158.75 77.851) (width 0.25) (layer "B.Cu") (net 21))
 (segment (start 167.64 80.264) (end 167.64 81.788) (width 0.25) (layer "B.Cu") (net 17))
 (segment (start 167.64 81.788) (end 171.45 85.598) (width 0.25) (layer "B.Cu") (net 17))
 (segment (start 171.45 96.266) (end 170.18 97.536) (width 0.25) (layer "B.Cu") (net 17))
 (segment (start 171.45 85.598) (end 171.45 96.266) (width 0.25) (layer "B.Cu") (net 17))
 (segment (start 129.54 82.169) (end 131.064 83.693) (width 0.25) (layer "B.Cu") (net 3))
 (segment (start 129.54 80.264) (end 129.54 82.169) (width 0.25) (layer "B.Cu") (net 3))
 (segment (start 131.064 83.693) (end 131.064 90.932) (width 0.25) (layer "B.Cu") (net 3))
 (segment (start 131.064 90.932) (end 129.54 92.456) (width 0.25) (layer "B.Cu") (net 3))
 (segment (start 129.54 92.456) (end 129.54 94.996) (width 0.25) (layer "B.Cu") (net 3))
 (segment (start 148.59 83.82) (end 153.67 88.9) (width 0.25) (layer "F.Cu") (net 24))
 (segment (start 157.48 65.024) (end 157.48 73.66) (width 0.25) (layer "F.Cu") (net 24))
 (segment (start 153.67 88.9) (end 153.67 96.266) (width 0.25) (layer "F.Cu") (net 24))
 (segment (start 157.48 73.66) (end 153.035 78.105) (width 0.25) (layer "F.Cu") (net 24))
 (segment (start 148.59 78.74) (end 148.59 83.82) (width 0.25) (layer "F.Cu") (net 24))
 (segment (start 149.225 78.105) (end 148.59 78.74) (width 0.25) (layer "F.Cu") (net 24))
 (segment (start 153.67 96.266) (end 154.94 97.536) (width 0.25) (layer "F.Cu") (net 24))
 (segment (start 153.035 78.105) (end 149.225 78.105) (width 0.25) (layer "F.Cu") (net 24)))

